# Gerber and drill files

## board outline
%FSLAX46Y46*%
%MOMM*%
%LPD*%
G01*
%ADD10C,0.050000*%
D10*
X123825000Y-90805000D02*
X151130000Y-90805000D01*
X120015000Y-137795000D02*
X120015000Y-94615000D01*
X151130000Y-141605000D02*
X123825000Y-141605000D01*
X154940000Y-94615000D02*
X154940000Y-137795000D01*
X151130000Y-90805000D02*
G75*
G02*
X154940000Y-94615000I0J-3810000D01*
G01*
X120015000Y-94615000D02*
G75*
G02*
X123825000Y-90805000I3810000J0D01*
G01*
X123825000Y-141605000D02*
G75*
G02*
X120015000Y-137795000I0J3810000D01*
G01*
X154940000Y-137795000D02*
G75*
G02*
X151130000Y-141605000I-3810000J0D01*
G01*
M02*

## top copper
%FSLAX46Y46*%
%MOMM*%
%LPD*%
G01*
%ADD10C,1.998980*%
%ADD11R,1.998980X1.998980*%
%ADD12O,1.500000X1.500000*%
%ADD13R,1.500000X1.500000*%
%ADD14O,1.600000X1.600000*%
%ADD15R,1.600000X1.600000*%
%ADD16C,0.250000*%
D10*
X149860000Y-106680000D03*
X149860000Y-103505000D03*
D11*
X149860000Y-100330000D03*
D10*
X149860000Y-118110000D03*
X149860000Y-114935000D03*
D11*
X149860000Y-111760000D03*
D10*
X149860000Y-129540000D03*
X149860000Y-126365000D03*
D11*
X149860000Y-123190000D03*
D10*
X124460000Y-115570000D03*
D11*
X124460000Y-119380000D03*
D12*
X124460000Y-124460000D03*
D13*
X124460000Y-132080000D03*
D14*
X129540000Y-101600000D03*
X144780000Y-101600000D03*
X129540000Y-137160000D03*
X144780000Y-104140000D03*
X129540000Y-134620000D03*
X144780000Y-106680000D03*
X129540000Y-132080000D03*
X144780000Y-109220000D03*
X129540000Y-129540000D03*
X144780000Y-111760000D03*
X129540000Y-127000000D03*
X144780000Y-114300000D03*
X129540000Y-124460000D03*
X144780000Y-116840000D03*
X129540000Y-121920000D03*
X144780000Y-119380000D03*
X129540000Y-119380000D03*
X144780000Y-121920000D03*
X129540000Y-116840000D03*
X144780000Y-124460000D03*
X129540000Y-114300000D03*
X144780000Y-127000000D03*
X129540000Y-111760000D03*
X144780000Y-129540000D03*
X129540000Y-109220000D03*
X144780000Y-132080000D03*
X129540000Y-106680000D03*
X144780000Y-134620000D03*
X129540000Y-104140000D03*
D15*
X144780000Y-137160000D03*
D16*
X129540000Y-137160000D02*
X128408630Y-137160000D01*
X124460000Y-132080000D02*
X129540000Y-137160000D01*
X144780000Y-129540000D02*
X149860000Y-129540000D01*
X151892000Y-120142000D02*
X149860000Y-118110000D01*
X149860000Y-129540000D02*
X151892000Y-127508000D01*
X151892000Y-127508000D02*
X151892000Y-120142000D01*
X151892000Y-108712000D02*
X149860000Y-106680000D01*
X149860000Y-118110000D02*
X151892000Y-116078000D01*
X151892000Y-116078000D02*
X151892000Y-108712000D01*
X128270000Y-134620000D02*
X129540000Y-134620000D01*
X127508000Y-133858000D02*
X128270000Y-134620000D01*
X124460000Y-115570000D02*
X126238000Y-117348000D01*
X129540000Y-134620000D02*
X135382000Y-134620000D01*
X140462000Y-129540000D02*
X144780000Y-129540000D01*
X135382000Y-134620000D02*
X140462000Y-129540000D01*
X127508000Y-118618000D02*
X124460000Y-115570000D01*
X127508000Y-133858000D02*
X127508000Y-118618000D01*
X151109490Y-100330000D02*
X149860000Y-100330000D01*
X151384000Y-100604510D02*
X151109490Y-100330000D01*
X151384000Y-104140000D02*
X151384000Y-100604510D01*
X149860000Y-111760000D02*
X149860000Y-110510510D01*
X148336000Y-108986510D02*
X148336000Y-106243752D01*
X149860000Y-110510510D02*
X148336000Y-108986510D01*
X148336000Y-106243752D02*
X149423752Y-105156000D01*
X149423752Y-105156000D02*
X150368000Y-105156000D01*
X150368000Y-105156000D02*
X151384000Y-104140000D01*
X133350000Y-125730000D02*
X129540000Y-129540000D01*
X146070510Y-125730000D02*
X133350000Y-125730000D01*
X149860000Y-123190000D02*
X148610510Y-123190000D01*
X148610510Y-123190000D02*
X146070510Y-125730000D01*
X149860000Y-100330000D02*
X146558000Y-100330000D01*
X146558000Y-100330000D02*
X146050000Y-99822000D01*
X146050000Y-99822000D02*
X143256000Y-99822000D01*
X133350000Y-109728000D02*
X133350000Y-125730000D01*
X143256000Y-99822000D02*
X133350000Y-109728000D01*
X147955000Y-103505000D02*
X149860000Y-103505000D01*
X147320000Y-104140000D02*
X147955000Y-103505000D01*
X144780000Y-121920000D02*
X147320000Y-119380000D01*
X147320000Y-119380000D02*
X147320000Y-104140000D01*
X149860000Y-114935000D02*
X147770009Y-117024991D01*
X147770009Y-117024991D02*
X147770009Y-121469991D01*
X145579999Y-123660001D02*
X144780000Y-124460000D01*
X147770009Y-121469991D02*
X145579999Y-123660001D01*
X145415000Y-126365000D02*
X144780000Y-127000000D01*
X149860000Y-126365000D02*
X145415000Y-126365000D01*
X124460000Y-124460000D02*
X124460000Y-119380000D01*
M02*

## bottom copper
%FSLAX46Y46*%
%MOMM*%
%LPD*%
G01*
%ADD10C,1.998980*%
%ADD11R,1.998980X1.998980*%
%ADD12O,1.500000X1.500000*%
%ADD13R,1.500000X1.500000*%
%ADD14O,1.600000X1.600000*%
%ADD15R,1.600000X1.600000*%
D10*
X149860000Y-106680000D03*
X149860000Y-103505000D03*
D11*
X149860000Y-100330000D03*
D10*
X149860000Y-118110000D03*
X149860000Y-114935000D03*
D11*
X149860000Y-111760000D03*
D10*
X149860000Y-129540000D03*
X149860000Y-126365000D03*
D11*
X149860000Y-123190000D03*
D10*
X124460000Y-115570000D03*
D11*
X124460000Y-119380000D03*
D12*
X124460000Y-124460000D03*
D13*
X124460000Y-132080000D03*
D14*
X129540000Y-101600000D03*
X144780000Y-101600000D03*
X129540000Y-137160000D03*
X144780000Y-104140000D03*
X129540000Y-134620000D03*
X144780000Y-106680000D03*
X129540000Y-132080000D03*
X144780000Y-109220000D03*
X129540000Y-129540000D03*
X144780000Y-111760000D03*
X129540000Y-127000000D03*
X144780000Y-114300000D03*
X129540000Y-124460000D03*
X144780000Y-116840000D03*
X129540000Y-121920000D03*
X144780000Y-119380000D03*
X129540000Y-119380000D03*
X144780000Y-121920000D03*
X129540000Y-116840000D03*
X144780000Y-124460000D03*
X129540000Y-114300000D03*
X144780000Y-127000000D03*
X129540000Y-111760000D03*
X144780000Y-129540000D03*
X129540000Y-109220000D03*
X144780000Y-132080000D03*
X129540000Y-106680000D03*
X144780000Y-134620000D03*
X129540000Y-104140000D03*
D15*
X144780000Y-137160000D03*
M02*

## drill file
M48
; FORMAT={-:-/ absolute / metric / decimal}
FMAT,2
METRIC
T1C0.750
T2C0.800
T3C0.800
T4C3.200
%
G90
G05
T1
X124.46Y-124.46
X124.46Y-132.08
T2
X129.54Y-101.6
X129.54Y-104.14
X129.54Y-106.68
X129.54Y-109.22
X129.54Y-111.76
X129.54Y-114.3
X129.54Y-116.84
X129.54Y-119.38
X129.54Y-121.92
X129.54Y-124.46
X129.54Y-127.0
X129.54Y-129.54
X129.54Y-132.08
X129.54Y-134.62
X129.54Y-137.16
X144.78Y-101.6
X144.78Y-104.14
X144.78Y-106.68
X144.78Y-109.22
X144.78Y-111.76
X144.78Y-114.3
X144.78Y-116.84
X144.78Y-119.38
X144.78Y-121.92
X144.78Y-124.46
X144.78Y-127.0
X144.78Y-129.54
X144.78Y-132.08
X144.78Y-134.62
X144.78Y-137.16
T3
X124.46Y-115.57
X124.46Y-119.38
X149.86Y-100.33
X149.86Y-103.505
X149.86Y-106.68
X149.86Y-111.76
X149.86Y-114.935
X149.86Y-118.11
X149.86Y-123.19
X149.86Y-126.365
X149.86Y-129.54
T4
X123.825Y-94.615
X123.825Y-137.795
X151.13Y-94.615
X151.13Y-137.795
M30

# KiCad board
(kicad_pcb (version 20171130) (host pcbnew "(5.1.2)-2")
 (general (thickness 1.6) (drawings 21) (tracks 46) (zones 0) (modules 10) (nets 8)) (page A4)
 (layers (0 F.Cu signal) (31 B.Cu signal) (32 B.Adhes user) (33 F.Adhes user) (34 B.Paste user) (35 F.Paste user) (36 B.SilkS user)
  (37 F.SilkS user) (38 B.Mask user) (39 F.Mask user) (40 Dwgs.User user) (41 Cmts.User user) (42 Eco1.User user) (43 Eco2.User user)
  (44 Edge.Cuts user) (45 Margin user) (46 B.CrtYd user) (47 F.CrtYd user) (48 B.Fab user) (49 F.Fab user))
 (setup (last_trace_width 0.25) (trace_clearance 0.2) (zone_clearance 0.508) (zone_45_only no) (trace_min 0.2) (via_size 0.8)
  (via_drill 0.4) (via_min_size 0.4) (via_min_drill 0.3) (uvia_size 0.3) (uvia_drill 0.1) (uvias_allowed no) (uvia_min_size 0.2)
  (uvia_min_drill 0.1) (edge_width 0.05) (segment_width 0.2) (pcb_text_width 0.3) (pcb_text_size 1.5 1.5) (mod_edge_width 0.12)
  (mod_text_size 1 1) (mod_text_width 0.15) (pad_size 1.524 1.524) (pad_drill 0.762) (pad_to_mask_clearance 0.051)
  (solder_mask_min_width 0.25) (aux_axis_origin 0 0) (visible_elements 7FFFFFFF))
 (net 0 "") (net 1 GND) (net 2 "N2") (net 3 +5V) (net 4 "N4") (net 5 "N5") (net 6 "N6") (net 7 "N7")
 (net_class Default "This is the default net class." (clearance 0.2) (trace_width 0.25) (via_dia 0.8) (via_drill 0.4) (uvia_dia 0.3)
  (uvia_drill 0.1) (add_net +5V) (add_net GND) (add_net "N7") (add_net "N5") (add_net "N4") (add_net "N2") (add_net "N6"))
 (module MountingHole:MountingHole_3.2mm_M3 (layer F.Cu) (at 123.825 94.615)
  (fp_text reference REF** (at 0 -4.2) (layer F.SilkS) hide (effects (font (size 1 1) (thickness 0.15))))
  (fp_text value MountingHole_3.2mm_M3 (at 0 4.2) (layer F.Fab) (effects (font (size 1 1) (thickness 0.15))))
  (pad 1 np_thru_hole circle (at 0 0) (size 3.2 3.2) (drill 3.2) (layers *.Cu *.Mask)))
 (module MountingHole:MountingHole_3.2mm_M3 (layer F.Cu) (at 123.825 137.795)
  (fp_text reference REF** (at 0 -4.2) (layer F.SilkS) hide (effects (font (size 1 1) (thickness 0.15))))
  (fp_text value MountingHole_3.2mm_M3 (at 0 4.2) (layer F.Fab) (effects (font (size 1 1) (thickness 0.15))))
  (pad 1 np_thru_hole circle (at 0 0) (size 3.2 3.2) (drill 3.2) (layers *.Cu *.Mask)))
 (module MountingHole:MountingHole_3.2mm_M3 (layer F.Cu) (at 151.13 94.615)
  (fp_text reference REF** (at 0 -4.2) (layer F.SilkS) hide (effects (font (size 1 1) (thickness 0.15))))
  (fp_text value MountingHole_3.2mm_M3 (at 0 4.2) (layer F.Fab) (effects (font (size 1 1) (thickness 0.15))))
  (pad 1 np_thru_hole circle (at 0 0) (size 3.2 3.2) (drill 3.2) (layers *.Cu *.Mask)))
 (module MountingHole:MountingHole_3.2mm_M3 (layer F.Cu) (at 151.13 137.795)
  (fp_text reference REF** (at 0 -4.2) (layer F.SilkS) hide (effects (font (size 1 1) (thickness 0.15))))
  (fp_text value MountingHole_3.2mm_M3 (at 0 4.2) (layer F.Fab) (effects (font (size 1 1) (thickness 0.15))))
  (pad 1 np_thru_hole circle (at 0 0) (size 3.2 3.2) (drill 3.2) (layers *.Cu *.Mask)))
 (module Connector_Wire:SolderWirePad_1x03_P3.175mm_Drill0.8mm (layer F.Cu) (at 149.86 100.33 270)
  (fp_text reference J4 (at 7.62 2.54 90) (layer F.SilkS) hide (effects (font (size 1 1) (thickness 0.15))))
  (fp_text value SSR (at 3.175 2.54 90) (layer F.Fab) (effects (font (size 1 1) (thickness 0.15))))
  (pad 3 thru_hole circle (at 6.35 0 270) (size 1.99898 1.99898) (drill 0.8001) (layers *.Cu *.Mask) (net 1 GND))
  (pad 2 thru_hole circle (at 3.175 0 270) (size 1.99898 1.99898) (drill 0.8001) (layers *.Cu *.Mask) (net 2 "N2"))
  (pad 1 thru_hole rect (at 0 0 270) (size 1.99898 1.99898) (drill 0.8001) (layers *.Cu *.Mask) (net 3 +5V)))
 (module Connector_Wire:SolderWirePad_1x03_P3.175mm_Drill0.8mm (layer F.Cu) (at 149.86 111.76 270)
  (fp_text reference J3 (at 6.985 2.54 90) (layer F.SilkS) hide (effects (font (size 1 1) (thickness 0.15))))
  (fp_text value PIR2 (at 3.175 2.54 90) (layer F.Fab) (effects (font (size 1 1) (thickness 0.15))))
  (pad 3 thru_hole circle (at 6.35 0 270) (size 1.99898 1.99898) (drill 0.8001) (layers *.Cu *.Mask) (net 1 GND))
  (pad 2 thru_hole circle (at 3.175 0 270) (size 1.99898 1.99898) (drill 0.8001) (layers *.Cu *.Mask) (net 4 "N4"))
  (pad 1 thru_hole rect (at 0 0 270) (size 1.99898 1.99898) (drill 0.8001) (layers *.Cu *.Mask) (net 3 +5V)))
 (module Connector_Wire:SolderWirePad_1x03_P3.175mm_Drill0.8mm (layer F.Cu) (at 149.86 123.19 270)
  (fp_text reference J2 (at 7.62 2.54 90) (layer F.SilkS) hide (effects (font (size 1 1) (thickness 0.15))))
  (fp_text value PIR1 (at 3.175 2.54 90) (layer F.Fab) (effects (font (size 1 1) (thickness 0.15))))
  (pad 3 thru_hole circle (at 6.35 0 270) (size 1.99898 1.99898) (drill 0.8001) (layers *.Cu *.Mask) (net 1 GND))
  (pad 2 thru_hole circle (at 3.175 0 270) (size 1.99898 1.99898) (drill 0.8001) (layers *.Cu *.Mask) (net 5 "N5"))
  (pad 1 thru_hole rect (at 0 0 270) (size 1.99898 1.99898) (drill 0.8001) (layers *.Cu *.Mask) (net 3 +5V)))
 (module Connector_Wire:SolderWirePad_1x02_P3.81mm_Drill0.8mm (layer F.Cu) (at 124.46 119.38 90)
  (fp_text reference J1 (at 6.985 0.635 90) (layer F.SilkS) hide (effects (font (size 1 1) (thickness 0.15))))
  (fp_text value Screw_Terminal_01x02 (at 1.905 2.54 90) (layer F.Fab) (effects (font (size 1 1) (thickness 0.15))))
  (pad 2 thru_hole circle (at 3.81 0 90) (size 1.99898 1.99898) (drill 0.8001) (layers *.Cu *.Mask) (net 1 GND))
  (pad 1 thru_hole rect (at 0 0 90) (size 1.99898 1.99898) (drill 0.8001) (layers *.Cu *.Mask) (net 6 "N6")))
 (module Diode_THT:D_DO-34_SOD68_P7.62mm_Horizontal (layer F.Cu) (at 124.46 132.08 90)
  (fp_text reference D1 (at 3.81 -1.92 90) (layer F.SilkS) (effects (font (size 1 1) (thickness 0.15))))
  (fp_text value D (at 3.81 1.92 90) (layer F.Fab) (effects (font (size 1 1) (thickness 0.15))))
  (pad 2 thru_hole oval (at 7.62 0 90) (size 1.5 1.5) (drill 0.75) (layers *.Cu *.Mask) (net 6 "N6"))
  (pad 1 thru_hole rect (at 0 0 90) (size 1.5 1.5) (drill 0.75) (layers *.Cu *.Mask) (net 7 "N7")))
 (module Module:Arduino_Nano (layer F.Cu) (at 144.78 137.16 180)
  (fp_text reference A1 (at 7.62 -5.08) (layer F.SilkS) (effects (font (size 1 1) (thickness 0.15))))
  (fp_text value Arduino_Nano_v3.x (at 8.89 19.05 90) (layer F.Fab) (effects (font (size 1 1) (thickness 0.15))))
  (pad 16 thru_hole oval (at 15.24 35.56 180) (size 1.6 1.6) (drill 0.8) (layers *.Cu *.Mask))
  (pad 15 thru_hole oval (at 0 35.56 180) (size 1.6 1.6) (drill 0.8) (layers *.Cu *.Mask))
  (pad 30 thru_hole oval (at 15.24 0 180) (size 1.6 1.6) (drill 0.8) (layers *.Cu *.Mask) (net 7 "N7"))
  (pad 14 thru_hole oval (at 0 33.02 180) (size 1.6 1.6) (drill 0.8) (layers *.Cu *.Mask))
  (pad 29 thru_hole oval (at 15.24 2.54 180) (size 1.6 1.6) (drill 0.8) (layers *.Cu *.Mask) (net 1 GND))
  (pad 13 thru_hole oval (at 0 30.48 180) (size 1.6 1.6) (drill 0.8) (layers *.Cu *.Mask))
  (pad 28 thru_hole oval (at 15.24 5.08 180) (size 1.6 1.6) (drill 0.8) (layers *.Cu *.Mask))
  (pad 12 thru_hole oval (at 0 27.94 180) (size 1.6 1.6) (drill 0.8) (layers *.Cu *.Mask))
  (pad 27 thru_hole oval (at 15.24 7.62 180) (size 1.6 1.6) (drill 0.8) (layers *.Cu *.Mask) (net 3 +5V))
  (pad 11 thru_hole oval (at 0 25.4 180) (size 1.6 1.6) (drill 0.8) (layers *.Cu *.Mask))
  (pad 26 thru_hole oval (at 15.24 10.16 180) (size 1.6 1.6) (drill 0.8) (layers *.Cu *.Mask))
  (pad 10 thru_hole oval (at 0 22.86 180) (size 1.6 1.6) (drill 0.8) (layers *.Cu *.Mask))
  (pad 25 thru_hole oval (at 15.24 12.7 180) (size 1.6 1.6) (drill 0.8) (layers *.Cu *.Mask))
  (pad 9 thru_hole oval (at 0 20.32 180) (size 1.6 1.6) (drill 0.8) (layers *.Cu *.Mask))
  (pad 24 thru_hole oval (at 15.24 15.24 180) (size 1.6 1.6) (drill 0.8) (layers *.Cu *.Mask))
  (pad 8 thru_hole oval (at 0 17.78 180) (size 1.6 1.6) (drill 0.8) (layers *.Cu *.Mask))
  (pad 23 thru_hole oval (at 15.24 17.78 180) (size 1.6 1.6) (drill 0.8) (layers *.Cu *.Mask))
  (pad 7 thru_hole oval (at 0 15.24 180) (size 1.6 1.6) (drill 0.8) (layers *.Cu *.Mask) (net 2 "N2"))
  (pad 22 thru_hole oval (at 15.24 20.32 180) (size 1.6 1.6) (drill 0.8) (layers *.Cu *.Mask))
  (pad 6 thru_hole oval (at 0 12.7 180) (size 1.6 1.6) (drill 0.8) (layers *.Cu *.Mask) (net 4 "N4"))
  (pad 21 thru_hole oval (at 15.24 22.86 180) (size 1.6 1.6) (drill 0.8) (layers *.Cu *.Mask))
  (pad 5 thru_hole oval (at 0 10.16 180) (size 1.6 1.6) (drill 0.8) (layers *.Cu *.Mask) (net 5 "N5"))
  (pad 20 thru_hole oval (at 15.24 25.4 180) (size 1.6 1.6) (drill 0.8) (layers *.Cu *.Mask))
  (pad 4 thru_hole oval (at 0 7.62 180) (size 1.6 1.6) (drill 0.8) (layers *.Cu *.Mask) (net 1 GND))
  (pad 19 thru_hole oval (at 15.24 27.94 180) (size 1.6 1.6) (drill 0.8) (layers *.Cu *.Mask))
  (pad 3 thru_hole oval (at 0 5.08 180) (size 1.6 1.6) (drill 0.8) (layers *.Cu *.Mask))
  (pad 18 thru_hole oval (at 15.24 30.48 180) (size 1.6 1.6) (drill 0.8) (layers *.Cu *.Mask))
  (pad 2 thru_hole oval (at 0 2.54 180) (size 1.6 1.6) (drill 0.8) (layers *.Cu *.Mask))
  (pad 17 thru_hole oval (at 15.24 33.02 180) (size 1.6 1.6) (drill 0.8) (layers *.Cu *.Mask))
  (pad 1 thru_hole rect (at 0 0 180) (size 1.6 1.6) (drill 0.8) (layers *.Cu *.Mask)))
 (gr_line (start 123.825 90.805) (end 151.13 90.805) (layer Edge.Cuts) (width 0.05))
 (gr_line (start 120.015 137.795) (end 120.015 94.615) (layer Edge.Cuts) (width 0.05))
 (gr_line (start 151.13 141.605) (end 123.825 141.605) (layer Edge.Cuts) (width 0.05))
 (gr_line (start 154.94 94.615) (end 154.94 137.795) (layer Edge.Cuts) (width 0.05))
 (gr_arc (start 151.13 94.615) (end 154.94 94.615) (angle -90) (layer Edge.Cuts) (width 0.05))
 (gr_arc (start 123.825 94.615) (end 123.825 90.805) (angle -90) (layer Edge.Cuts) (width 0.05))
 (gr_arc (start 123.825 137.795) (end 120.015 137.795) (angle -90) (layer Edge.Cuts) (width 0.05))
 (gr_arc (start 151.13 137.795) (end 151.13 141.605) (angle -90) (layer Edge.Cuts) (width 0.05))
 (segment (start 129.54 137.16) (end 128.40863 137.16) (width 0.25) (layer F.Cu) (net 7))
 (segment (start 124.46 132.08) (end 129.54 137.16) (width 0.25) (layer F.Cu) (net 7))
 (segment (start 144.78 129.54) (end 149.86 129.54) (width 0.25) (layer F.Cu) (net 1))
 (segment (start 151.892 120.142) (end 149.86 118.11) (width 0.25) (layer F.Cu) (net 1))
 (segment (start 149.86 129.54) (end 151.892 127.508) (width 0.25) (layer F.Cu) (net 1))
 (segment (start 151.892 127.508) (end 151.892 120.142) (width 0.25) (layer F.Cu) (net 1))
 (segment (start 151.892 108.712) (end 149.86 106.68) (width 0.25) (layer F.Cu) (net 1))
 (segment (start 149.86 118.11) (end 151.892 116.078) (width 0.25) (layer F.Cu) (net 1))
 (segment (start 151.892 116.078) (end 151.892 108.712) (width 0.25) (layer F.Cu) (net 1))
 (segment (start 128.27 134.62) (end 129.54 134.62) (width 0.25) (layer F.Cu) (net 1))
 (segment (start 127.508 133.858) (end 128.27 134.62) (width 0.25) (layer F.Cu) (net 1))
 (segment (start 124.46 115.57) (end 126.238 117.348) (width 0.25) (layer F.Cu) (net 1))
 (segment (start 129.54 134.62) (end 135.382 134.62) (width 0.25) (layer F.Cu) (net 1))
 (segment (start 140.462 129.54) (end 144.78 129.54) (width 0.25) (layer F.Cu) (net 1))
 (segment (start 135.382 134.62) (end 140.462 129.54) (width 0.25) (layer F.Cu) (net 1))
 (segment (start 127.508 118.618) (end 124.46 115.57) (width 0.25) (layer F.Cu) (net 1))
 (segment (start 127.508 133.858) (end 127.508 118.618) (width 0.25) (layer F.Cu) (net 1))
 (segment (start 151.10949 100.33) (end 149.86 100.33) (width 0.25) (layer F.Cu) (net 3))
 (segment (start 151.384 100.60451) (end 151.10949 100.33) (width 0.25) (layer F.Cu) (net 3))
 (segment (start 151.384 104.14) (end 151.384 100.60451) (width 0.25) (layer F.Cu) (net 3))
 (segment (start 149.86 111.76) (end 149.86 110.51051) (width 0.25) (layer F.Cu) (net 3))
 (segment (start 148.336 108.98651) (end 148.336 106.243752) (width 0.25) (layer F.Cu) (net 3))
 (segment (start 149.86 110.51051) (end 148.336 108.98651) (width 0.25) (layer F.Cu) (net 3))
 (segment (start 148.336 106.243752) (end 149.423752 105.156) (width 0.25) (layer F.Cu) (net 3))
 (segment (start 149.423752 105.156) (end 150.368 105.156) (width 0.25) (layer F.Cu) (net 3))
 (segment (start 150.368 105.156) (end 151.384 104.14) (width 0.25) (layer F.Cu) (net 3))
 (segment (start 133.35 125.73) (end 129.54 129.54) (width 0.25) (layer F.Cu) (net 3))
 (segment (start 146.07051 125.73) (end 133.35 125.73) (width 0.25) (layer F.Cu) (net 3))
 (segment (start 149.86 123.19) (end 148.61051 123.19) (width 0.25) (layer F.Cu) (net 3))
 (segment (start 148.61051 123.19) (end 146.07051 125.73) (width 0.25) (layer F.Cu) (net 3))
 (segment (start 149.86 100.33) (end 146.558 100.33) (width 0.25) (layer F.Cu) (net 3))
 (segment (start 146.558 100.33) (end 146.05 99.822) (width 0.25) (layer F.Cu) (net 3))
 (segment (start 146.05 99.822) (end 143.256 99.822) (width 0.25) (layer F.Cu) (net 3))
 (segment (start 133.35 109.728) (end 133.35 125.73) (width 0.25) (layer F.Cu) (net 3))
 (segment (start 143.256 99.822) (end 133.35 109.728) (width 0.25) (layer F.Cu) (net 3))
 (segment (start 147.955 103.505) (end 149.86 103.505) (width 0.25) (layer F.Cu) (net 2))
 (segment (start 147.32 104.14) (end 147.955 103.505) (width 0.25) (layer F.Cu) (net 2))
 (segment (start 144.78 121.92) (end 147.32 119.38) (width 0.25) (layer F.Cu) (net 2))
 (segment (start 147.32 119.38) (end 147.32 104.14) (width 0.25) (layer F.Cu) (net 2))
 (segment (start 149.86 114.935) (end 147.770009 117.024991) (width 0.25) (layer F.Cu) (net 4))
 (segment (start 147.770009 117.024991) (end 147.770009 121.469991) (width 0.25) (layer F.Cu) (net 4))
 (segment (start 145.579999 123.660001) (end 144.78 124.46) (width 0.25) (layer F.Cu) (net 4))
 (segment (start 147.770009 121.469991) (end 145.579999 123.660001) (width 0.25) (layer F.Cu) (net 4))
 (segment (start 145.415 126.365) (end 144.78 127) (width 0.25) (layer F.Cu) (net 5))
 (segment (start 149.86 126.365) (end 145.415 126.365) (width 0.25) (layer F.Cu) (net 5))
 (segment (start 124.46 124.46) (end 124.46 119.38) (width 0.25) (layer F.Cu) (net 6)))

